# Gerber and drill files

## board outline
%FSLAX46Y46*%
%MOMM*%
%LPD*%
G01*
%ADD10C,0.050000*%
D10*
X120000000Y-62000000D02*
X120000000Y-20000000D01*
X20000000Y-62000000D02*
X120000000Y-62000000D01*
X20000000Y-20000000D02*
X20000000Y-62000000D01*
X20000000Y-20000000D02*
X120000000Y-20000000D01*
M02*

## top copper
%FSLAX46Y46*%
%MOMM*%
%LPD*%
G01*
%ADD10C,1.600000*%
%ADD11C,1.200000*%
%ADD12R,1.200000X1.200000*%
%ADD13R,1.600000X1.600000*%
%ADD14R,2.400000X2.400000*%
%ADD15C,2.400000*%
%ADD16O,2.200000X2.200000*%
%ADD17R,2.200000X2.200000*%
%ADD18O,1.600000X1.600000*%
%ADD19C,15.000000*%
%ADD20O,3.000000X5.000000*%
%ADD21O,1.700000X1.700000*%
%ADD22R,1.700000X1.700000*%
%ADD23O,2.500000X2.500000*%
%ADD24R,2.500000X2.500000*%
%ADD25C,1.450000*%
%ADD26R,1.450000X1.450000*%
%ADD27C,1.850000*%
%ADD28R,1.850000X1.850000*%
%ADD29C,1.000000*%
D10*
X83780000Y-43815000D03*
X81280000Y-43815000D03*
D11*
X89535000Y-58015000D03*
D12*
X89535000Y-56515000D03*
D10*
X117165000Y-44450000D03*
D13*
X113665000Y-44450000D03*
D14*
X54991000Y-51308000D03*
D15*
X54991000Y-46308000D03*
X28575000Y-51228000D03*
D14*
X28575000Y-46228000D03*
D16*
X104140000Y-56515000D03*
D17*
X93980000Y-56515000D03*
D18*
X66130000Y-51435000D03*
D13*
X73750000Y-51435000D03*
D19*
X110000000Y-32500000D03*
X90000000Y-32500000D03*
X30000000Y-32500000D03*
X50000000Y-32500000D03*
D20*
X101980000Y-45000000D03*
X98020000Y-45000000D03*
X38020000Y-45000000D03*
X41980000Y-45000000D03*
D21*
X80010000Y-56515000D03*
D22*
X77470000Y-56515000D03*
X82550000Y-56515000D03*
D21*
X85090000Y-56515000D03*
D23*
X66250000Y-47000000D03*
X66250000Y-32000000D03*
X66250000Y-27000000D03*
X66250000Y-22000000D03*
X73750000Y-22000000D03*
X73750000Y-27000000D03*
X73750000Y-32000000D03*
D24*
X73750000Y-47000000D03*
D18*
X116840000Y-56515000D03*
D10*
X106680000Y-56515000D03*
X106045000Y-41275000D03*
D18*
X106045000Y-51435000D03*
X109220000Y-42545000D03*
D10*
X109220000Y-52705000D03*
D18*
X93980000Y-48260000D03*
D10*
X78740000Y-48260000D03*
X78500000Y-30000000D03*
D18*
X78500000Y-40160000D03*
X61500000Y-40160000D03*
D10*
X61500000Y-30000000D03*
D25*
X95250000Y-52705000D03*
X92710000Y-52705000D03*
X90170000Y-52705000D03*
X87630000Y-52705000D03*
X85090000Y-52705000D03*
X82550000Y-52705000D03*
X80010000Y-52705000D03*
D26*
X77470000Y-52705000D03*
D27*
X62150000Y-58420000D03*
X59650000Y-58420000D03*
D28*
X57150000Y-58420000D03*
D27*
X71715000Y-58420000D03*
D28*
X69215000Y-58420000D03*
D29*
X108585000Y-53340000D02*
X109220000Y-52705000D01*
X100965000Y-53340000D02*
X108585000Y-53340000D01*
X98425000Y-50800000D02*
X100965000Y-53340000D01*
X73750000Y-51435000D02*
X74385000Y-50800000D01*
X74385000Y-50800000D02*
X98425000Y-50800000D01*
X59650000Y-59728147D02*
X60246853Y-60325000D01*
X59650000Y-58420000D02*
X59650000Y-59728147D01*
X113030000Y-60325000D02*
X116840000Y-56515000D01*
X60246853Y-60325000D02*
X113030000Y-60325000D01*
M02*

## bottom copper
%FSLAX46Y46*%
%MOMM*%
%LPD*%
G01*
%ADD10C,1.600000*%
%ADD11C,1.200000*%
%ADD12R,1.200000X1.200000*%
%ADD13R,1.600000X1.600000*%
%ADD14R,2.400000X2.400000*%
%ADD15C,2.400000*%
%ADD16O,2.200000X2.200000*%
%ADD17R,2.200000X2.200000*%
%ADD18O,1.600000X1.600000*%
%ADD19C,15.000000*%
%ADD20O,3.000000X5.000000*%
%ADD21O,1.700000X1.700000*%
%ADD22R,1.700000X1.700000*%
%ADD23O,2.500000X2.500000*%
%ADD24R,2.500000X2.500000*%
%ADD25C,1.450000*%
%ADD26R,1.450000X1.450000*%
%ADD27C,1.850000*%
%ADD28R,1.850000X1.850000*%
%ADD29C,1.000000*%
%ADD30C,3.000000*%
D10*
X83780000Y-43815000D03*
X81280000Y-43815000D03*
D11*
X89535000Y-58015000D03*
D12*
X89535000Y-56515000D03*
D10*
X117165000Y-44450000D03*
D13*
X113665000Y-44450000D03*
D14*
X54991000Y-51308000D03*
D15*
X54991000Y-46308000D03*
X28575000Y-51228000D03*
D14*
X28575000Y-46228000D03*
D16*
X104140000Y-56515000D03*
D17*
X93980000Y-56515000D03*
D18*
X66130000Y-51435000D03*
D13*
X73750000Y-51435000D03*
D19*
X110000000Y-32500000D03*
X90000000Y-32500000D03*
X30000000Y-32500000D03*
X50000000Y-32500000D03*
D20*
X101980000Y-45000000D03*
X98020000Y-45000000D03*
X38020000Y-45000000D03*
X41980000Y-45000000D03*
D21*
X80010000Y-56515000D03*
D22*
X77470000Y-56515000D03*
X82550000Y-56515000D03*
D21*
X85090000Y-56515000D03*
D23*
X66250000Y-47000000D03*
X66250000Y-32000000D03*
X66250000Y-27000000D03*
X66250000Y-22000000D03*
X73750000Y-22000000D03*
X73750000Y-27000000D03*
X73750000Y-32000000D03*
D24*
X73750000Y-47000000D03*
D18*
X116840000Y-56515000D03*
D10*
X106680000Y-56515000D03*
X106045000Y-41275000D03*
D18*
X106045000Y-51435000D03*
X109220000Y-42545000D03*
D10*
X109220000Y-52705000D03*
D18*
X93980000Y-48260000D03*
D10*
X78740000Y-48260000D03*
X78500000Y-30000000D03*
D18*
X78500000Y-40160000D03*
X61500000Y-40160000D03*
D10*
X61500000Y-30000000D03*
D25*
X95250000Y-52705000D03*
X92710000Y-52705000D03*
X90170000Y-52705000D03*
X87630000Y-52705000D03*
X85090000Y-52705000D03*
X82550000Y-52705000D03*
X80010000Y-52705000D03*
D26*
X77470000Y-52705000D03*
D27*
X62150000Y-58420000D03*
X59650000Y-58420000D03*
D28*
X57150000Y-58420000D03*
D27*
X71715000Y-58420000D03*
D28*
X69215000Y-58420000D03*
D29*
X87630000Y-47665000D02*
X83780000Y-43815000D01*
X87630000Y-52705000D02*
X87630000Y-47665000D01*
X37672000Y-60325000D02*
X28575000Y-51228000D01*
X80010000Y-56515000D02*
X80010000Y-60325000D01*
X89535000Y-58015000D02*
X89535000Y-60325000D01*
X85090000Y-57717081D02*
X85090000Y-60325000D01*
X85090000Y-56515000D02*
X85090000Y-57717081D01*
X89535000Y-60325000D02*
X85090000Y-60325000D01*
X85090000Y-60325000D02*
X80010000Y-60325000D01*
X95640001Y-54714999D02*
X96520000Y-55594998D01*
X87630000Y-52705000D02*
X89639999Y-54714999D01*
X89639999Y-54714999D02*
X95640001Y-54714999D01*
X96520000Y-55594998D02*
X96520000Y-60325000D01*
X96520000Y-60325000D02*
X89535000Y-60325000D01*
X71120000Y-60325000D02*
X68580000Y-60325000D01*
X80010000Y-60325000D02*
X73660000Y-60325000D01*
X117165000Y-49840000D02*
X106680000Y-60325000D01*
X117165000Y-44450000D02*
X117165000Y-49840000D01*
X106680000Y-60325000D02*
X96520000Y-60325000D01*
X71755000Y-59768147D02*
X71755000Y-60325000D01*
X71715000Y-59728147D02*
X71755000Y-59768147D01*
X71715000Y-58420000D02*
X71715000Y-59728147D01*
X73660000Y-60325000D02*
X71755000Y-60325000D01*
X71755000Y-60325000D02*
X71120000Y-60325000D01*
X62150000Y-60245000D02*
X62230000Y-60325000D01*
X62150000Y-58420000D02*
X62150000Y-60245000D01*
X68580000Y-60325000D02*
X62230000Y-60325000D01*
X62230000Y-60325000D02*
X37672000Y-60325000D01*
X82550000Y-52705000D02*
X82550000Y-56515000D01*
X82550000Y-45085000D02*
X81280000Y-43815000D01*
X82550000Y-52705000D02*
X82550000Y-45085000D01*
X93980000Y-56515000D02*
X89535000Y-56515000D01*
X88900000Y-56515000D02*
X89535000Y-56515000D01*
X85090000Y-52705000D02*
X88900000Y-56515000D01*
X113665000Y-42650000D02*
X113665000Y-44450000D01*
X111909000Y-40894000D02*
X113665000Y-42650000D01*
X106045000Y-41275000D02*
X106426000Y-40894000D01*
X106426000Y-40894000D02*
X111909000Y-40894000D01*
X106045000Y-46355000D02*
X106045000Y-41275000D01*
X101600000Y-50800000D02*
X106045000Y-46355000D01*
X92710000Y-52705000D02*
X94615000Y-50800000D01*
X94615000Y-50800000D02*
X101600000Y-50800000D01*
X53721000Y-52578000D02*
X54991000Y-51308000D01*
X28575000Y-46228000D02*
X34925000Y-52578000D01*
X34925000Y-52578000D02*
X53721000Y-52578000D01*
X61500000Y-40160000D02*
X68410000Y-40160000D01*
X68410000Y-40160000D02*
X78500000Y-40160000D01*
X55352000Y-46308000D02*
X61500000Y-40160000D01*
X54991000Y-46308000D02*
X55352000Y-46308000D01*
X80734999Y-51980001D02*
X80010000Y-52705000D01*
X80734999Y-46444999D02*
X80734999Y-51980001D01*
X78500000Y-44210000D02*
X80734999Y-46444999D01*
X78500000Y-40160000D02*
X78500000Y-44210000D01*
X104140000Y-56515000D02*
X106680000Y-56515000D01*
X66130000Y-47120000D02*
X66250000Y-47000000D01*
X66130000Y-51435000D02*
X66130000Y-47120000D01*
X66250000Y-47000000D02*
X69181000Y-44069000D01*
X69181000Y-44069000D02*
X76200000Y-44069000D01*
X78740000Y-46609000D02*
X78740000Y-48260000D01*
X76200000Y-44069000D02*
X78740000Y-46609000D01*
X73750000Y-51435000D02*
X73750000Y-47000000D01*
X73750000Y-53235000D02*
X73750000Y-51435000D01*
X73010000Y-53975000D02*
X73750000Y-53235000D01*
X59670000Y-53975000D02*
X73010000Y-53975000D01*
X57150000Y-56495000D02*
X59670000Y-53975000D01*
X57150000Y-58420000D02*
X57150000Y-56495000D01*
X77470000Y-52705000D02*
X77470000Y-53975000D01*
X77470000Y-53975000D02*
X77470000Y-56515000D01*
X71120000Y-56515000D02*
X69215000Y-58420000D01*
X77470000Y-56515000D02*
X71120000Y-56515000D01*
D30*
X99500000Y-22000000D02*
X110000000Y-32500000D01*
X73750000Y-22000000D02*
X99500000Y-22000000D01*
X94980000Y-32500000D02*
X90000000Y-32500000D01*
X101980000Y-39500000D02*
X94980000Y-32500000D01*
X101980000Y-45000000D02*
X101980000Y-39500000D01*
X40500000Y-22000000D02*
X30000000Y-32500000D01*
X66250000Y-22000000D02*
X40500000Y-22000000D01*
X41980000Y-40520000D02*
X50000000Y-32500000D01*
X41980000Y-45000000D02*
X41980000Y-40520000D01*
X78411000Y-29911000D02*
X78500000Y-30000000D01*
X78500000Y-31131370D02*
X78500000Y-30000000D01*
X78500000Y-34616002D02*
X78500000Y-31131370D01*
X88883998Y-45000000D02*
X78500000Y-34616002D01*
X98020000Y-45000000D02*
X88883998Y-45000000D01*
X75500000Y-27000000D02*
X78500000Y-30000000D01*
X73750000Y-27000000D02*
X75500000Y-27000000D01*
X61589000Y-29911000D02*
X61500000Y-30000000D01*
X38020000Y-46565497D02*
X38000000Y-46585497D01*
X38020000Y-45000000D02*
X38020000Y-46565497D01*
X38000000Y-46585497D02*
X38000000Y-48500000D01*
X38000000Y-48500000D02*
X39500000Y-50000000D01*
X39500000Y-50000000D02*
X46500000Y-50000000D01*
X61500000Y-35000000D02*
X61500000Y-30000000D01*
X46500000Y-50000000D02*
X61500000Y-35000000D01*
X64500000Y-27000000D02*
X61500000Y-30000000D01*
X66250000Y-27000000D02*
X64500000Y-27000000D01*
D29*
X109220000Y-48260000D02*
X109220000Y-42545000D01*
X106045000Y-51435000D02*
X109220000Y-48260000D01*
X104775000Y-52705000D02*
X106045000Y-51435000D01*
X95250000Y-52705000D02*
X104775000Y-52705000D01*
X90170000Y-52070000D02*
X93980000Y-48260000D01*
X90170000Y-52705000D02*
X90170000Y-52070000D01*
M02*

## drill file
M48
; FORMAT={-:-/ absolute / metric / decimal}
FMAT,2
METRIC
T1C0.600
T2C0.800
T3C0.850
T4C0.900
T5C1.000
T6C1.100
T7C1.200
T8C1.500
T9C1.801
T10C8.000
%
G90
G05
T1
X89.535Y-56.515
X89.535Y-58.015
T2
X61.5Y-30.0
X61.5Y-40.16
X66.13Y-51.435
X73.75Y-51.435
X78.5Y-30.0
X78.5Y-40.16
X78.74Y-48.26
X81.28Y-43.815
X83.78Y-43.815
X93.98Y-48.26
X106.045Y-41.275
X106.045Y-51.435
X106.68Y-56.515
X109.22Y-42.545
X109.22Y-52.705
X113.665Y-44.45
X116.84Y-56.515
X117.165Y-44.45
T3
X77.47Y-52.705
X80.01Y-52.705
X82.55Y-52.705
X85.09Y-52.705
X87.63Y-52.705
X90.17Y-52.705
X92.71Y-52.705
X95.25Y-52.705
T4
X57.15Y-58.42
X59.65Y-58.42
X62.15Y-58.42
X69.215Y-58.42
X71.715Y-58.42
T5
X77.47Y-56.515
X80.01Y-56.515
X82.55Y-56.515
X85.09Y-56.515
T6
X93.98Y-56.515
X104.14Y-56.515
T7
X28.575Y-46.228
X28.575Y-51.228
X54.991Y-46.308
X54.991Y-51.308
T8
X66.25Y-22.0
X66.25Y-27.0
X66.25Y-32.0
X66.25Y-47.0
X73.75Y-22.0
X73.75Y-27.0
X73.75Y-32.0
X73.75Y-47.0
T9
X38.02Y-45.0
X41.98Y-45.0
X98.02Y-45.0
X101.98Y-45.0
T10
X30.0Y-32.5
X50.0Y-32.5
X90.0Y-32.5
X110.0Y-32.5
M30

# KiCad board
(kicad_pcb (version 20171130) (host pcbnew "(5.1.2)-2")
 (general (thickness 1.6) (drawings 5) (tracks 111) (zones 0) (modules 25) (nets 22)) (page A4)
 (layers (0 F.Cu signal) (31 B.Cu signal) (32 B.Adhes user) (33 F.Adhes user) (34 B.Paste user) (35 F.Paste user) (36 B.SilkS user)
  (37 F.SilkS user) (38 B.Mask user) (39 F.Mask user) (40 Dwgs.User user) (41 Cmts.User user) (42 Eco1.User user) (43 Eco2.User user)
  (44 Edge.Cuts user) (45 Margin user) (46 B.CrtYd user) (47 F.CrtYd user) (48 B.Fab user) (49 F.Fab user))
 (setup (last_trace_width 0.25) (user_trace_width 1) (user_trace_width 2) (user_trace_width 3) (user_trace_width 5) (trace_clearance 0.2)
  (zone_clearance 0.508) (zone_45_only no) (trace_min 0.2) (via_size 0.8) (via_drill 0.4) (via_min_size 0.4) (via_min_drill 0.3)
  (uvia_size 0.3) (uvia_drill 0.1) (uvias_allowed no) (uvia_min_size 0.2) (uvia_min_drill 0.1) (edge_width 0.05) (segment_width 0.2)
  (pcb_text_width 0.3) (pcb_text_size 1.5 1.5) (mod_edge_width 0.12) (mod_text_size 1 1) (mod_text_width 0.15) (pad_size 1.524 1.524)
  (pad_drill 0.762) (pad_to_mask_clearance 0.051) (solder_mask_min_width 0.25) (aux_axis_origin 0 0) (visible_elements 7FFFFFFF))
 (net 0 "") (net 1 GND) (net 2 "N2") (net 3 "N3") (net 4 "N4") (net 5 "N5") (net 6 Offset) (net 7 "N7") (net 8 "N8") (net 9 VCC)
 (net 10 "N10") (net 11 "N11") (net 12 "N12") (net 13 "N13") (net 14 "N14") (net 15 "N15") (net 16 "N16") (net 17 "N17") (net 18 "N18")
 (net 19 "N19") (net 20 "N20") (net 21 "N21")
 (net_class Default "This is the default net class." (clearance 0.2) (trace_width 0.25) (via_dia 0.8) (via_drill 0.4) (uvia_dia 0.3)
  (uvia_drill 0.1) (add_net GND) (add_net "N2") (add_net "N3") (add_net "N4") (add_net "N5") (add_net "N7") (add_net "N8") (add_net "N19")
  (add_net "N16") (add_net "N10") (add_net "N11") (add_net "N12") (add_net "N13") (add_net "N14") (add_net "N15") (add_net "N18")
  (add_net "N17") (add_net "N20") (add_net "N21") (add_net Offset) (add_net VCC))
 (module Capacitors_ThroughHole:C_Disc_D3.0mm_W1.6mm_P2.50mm (layer F.Cu) (at 81.28 43.815)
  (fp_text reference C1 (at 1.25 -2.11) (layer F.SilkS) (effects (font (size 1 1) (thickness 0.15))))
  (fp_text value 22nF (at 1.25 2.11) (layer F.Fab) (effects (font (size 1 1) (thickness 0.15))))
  (pad 2 thru_hole circle (at 2.5 0) (size 1.6 1.6) (drill 0.8) (layers *.Cu *.Mask) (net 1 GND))
  (pad 1 thru_hole circle (at 0 0) (size 1.6 1.6) (drill 0.8) (layers *.Cu *.Mask) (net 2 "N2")))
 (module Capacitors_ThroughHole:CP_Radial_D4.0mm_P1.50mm (layer F.Cu) (at 89.535 56.515 270)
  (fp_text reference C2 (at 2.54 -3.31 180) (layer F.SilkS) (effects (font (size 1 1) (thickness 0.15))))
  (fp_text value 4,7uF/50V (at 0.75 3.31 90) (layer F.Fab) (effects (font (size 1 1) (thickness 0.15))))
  (pad 2 thru_hole circle (at 1.5 0 270) (size 1.2 1.2) (drill 0.6) (layers *.Cu *.Mask) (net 1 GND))
  (pad 1 thru_hole rect (at 0 0 270) (size 1.2 1.2) (drill 0.6) (layers *.Cu *.Mask) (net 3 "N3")))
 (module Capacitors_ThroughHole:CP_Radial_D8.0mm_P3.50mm (layer F.Cu) (at 113.665 44.45)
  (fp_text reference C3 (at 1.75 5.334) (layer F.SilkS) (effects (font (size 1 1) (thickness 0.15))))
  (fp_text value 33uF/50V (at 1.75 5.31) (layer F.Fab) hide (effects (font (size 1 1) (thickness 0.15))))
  (pad 2 thru_hole circle (at 3.5 0) (size 1.6 1.6) (drill 0.8) (layers *.Cu *.Mask) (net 1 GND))
  (pad 1 thru_hole rect (at 0 0) (size 1.6 1.6) (drill 0.8) (layers *.Cu *.Mask) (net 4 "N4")))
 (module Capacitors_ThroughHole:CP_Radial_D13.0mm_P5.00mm (layer F.Cu) (at 54.991 51.308 90)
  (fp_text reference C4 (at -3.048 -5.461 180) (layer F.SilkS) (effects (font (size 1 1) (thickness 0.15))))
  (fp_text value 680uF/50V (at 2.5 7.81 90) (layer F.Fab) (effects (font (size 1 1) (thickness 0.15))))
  (pad 1 thru_hole rect (at 0 0 90) (size 2.4 2.4) (drill 1.2) (layers *.Cu *.Mask) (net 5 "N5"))
  (pad 2 thru_hole circle (at 5 0 90) (size 2.4 2.4) (drill 1.2) (layers *.Cu *.Mask) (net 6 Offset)))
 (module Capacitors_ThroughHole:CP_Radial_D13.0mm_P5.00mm (layer F.Cu) (at 28.575 46.228 270)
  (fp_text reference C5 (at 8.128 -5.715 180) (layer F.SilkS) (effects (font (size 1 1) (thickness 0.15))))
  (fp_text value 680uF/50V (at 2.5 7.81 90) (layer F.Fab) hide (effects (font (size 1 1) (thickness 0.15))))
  (pad 2 thru_hole circle (at 5 0 270) (size 2.4 2.4) (drill 1.2) (layers *.Cu *.Mask) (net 1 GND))
  (pad 1 thru_hole rect (at 0 0 270) (size 2.4 2.4) (drill 1.2) (layers *.Cu *.Mask) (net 5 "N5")))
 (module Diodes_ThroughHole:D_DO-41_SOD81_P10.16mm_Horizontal (layer F.Cu) (at 93.98 56.515)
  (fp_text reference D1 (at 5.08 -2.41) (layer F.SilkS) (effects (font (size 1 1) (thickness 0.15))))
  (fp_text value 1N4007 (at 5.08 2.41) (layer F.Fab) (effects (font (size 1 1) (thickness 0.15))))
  (pad 2 thru_hole oval (at 10.16 0) (size 2.2 2.2) (drill 1.1) (layers *.Cu *.Mask) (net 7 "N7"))
  (pad 1 thru_hole rect (at 0 0) (size 2.2 2.2) (drill 1.1) (layers *.Cu *.Mask) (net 3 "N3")))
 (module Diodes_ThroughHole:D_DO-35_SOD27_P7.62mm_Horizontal (layer F.Cu) (at 73.75 51.435 180)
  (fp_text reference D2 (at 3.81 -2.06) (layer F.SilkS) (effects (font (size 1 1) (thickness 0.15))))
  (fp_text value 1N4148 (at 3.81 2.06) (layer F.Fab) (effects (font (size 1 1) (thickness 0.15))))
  (pad 2 thru_hole oval (at 7.62 0 180) (size 1.6 1.6) (drill 0.8) (layers *.Cu *.Mask) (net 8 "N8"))
  (pad 1 thru_hole rect (at 0 0 180) (size 1.6 1.6) (drill 0.8) (layers *.Cu *.Mask) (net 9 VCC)))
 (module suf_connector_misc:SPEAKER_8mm (layer F.Cu) (at 110 32.5)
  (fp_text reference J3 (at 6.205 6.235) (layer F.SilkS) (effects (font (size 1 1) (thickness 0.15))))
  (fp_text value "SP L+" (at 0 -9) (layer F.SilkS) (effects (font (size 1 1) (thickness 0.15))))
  (pad 1 thru_hole circle (at 0 0) (size 15 15) (drill 8) (layers *.Cu *.Mask) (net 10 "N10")))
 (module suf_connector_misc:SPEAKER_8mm (layer F.Cu) (at 90 32.5)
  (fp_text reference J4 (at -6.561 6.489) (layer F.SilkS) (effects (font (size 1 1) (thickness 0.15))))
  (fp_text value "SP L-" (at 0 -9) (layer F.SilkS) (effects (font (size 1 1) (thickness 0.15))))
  (pad 1 thru_hole circle (at 0 0) (size 15 15) (drill 8) (layers *.Cu *.Mask) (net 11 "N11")))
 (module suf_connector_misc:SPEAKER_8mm (layer F.Cu) (at 30 32.5)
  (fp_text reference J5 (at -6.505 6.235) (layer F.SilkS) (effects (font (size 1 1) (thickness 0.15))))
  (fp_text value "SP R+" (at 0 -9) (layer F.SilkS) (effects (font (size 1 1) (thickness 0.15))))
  (pad 1 thru_hole circle (at 0 0) (size 15 15) (drill 8) (layers *.Cu *.Mask) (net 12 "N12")))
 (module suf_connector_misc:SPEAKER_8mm (layer F.Cu) (at 50 32.5)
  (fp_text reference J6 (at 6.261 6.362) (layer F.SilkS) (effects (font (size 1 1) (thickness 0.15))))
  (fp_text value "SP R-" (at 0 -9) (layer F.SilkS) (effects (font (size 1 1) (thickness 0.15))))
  (pad 1 thru_hole circle (at 0 0) (size 15 15) (drill 8) (layers *.Cu *.Mask) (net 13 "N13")))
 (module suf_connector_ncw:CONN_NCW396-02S (layer F.Cu) (at 100 45)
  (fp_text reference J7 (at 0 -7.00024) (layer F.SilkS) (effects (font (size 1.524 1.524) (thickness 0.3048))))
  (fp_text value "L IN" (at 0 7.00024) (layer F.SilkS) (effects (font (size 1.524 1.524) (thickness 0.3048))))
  (pad 2 thru_hole oval (at 1.98 0) (size 3 5) (drill 1.80086) (layers *.Cu *.Mask F.SilkS) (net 11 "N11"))
  (pad 1 thru_hole oval (at -1.98 0) (size 3 5) (drill 1.80086) (layers *.Cu *.Mask F.SilkS) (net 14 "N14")))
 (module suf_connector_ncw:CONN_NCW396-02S (layer F.Cu) (at 40 45)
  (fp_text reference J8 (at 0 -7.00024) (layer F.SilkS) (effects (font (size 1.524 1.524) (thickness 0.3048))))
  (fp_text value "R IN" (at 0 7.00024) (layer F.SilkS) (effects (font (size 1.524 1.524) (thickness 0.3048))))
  (pad 1 thru_hole oval (at -1.98 0) (size 3 5) (drill 1.80086) (layers *.Cu *.Mask F.SilkS) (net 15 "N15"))
  (pad 2 thru_hole oval (at 1.98 0) (size 3 5) (drill 1.80086) (layers *.Cu *.Mask F.SilkS) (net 13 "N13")))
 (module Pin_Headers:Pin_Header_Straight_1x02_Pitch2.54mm (layer F.Cu) (at 77.47 56.515 90)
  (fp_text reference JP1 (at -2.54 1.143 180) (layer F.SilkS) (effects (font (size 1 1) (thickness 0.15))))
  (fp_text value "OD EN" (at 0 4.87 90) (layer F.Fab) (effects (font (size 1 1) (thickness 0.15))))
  (pad 2 thru_hole oval (at 0 2.54 90) (size 1.7 1.7) (drill 1) (layers *.Cu *.Mask) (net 1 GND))
  (pad 1 thru_hole rect (at 0 0 90) (size 1.7 1.7) (drill 1) (layers *.Cu *.Mask) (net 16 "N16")))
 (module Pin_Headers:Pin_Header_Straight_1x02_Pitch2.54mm (layer F.Cu) (at 82.55 56.515 90)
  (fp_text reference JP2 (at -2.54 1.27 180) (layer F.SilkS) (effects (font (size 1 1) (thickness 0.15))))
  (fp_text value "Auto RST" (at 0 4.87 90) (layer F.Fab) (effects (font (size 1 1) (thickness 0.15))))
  (pad 1 thru_hole rect (at 0 0 90) (size 1.7 1.7) (drill 1) (layers *.Cu *.Mask) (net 2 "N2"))
  (pad 2 thru_hole oval (at 0 2.54 90) (size 1.7 1.7) (drill 1) (layers *.Cu *.Mask) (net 1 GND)))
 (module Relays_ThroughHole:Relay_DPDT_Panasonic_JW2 (layer F.Cu) (at 73.75 47 180)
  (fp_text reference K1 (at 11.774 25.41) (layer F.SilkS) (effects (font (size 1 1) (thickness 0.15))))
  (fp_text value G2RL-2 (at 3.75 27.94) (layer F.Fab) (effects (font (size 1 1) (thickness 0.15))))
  (pad 8 thru_hole oval (at 7.5 0 180) (size 2.5 2.5) (drill 1.5) (layers *.Cu *.Mask) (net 8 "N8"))
  (pad 7 thru_hole oval (at 7.5 15 180) (size 2.5 2.5) (drill 1.5) (layers *.Cu *.Mask) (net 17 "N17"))
  (pad 6 thru_hole oval (at 7.5 20 180) (size 2.5 2.5) (drill 1.5) (layers *.Cu *.Mask) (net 15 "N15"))
  (pad 5 thru_hole oval (at 7.5 25 180) (size 2.5 2.5) (drill 1.5) (layers *.Cu *.Mask) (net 12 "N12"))
  (pad 4 thru_hole oval (at 0 25 180) (size 2.5 2.5) (drill 1.5) (layers *.Cu *.Mask) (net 10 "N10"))
  (pad 3 thru_hole oval (at 0 20 180) (size 2.5 2.5) (drill 1.5) (layers *.Cu *.Mask) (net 14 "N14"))
  (pad 2 thru_hole oval (at 0 15 180) (size 2.5 2.5) (drill 1.5) (layers *.Cu *.Mask) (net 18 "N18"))
  (pad 1 thru_hole rect (at 0 0 180) (size 2.5 2.5) (drill 1.5) (layers *.Cu *.Mask) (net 9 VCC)))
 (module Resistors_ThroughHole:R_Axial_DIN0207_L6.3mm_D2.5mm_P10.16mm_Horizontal (layer F.Cu) (at 106.68 56.515)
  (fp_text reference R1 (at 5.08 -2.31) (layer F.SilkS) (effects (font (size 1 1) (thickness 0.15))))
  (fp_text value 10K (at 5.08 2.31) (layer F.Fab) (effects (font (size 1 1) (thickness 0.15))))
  (pad 2 thru_hole oval (at 10.16 0) (size 1.6 1.6) (drill 0.8) (layers *.Cu *.Mask) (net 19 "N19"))
  (pad 1 thru_hole circle (at 0 0) (size 1.6 1.6) (drill 0.8) (layers *.Cu *.Mask) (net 7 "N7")))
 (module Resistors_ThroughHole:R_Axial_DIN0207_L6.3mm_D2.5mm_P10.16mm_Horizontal (layer F.Cu) (at 106.045 41.275 270)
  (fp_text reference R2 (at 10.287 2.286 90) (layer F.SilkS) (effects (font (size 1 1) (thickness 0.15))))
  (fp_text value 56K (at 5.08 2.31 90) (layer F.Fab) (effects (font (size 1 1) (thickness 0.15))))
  (pad 1 thru_hole circle (at 0 0 270) (size 1.6 1.6) (drill 0.8) (layers *.Cu *.Mask) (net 4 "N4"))
  (pad 2 thru_hole oval (at 10.16 0 270) (size 1.6 1.6) (drill 0.8) (layers *.Cu *.Mask) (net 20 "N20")))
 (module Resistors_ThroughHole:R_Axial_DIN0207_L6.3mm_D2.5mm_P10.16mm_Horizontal (layer F.Cu) (at 109.22 52.705 90)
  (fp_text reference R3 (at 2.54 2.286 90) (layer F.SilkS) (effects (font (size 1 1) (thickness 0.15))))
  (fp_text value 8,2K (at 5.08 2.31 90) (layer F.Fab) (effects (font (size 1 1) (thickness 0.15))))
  (pad 2 thru_hole oval (at 10.16 0 90) (size 1.6 1.6) (drill 0.8) (layers *.Cu *.Mask) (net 20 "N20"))
  (pad 1 thru_hole circle (at 0 0 90) (size 1.6 1.6) (drill 0.8) (layers *.Cu *.Mask) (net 9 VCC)))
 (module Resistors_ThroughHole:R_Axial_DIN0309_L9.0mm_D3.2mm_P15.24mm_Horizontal (layer F.Cu) (at 78.74 48.26)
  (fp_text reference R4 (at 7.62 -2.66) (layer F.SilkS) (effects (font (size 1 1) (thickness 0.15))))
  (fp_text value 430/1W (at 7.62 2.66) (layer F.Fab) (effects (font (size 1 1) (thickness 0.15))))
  (pad 2 thru_hole oval (at 15.24 0) (size 1.6 1.6) (drill 0.8) (layers *.Cu *.Mask) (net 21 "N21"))
  (pad 1 thru_hole circle (at 0 0) (size 1.6 1.6) (drill 0.8) (layers *.Cu *.Mask) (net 8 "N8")))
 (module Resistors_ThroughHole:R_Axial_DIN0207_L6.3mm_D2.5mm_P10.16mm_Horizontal (layer F.Cu) (at 78.5 30 270)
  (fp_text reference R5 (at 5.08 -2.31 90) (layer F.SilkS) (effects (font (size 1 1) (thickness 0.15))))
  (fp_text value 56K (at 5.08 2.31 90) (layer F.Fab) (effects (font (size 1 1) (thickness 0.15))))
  (pad 1 thru_hole circle (at 0 0 270) (size 1.6 1.6) (drill 0.8) (layers *.Cu *.Mask) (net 14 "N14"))
  (pad 2 thru_hole oval (at 10.16 0 270) (size 1.6 1.6) (drill 0.8) (layers *.Cu *.Mask) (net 6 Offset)))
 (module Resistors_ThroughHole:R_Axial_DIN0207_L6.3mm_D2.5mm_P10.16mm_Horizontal (layer F.Cu) (at 61.5 30 270)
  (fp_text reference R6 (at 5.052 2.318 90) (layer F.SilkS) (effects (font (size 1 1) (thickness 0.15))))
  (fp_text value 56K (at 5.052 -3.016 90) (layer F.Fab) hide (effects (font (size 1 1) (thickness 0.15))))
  (pad 2 thru_hole oval (at 10.16 0 270) (size 1.6 1.6) (drill 0.8) (layers *.Cu *.Mask) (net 6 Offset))
  (pad 1 thru_hole circle (at 0 0 270) (size 1.6 1.6) (drill 0.8) (layers *.Cu *.Mask) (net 15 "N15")))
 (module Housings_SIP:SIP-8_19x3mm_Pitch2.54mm (layer F.Cu) (at 77.47 52.705)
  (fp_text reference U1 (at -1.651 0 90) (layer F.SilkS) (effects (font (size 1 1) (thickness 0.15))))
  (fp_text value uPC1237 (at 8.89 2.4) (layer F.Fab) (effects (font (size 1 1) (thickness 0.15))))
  (pad 8 thru_hole circle (at 17.78 0 90) (size 1.45 1.45) (drill 0.85) (layers *.Cu *.Mask) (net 20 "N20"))
  (pad 7 thru_hole circle (at 15.24 0 90) (size 1.45 1.45) (drill 0.85) (layers *.Cu *.Mask) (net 4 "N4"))
  (pad 6 thru_hole circle (at 12.7 0 90) (size 1.45 1.45) (drill 0.85) (layers *.Cu *.Mask) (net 21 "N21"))
  (pad 5 thru_hole circle (at 10.16 0 90) (size 1.45 1.45) (drill 0.85) (layers *.Cu *.Mask) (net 1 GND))
  (pad 4 thru_hole circle (at 7.62 0 90) (size 1.45 1.45) (drill 0.85) (layers *.Cu *.Mask) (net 3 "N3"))
  (pad 3 thru_hole circle (at 5.08 0 90) (size 1.45 1.45) (drill 0.85) (layers *.Cu *.Mask) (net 2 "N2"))
  (pad 2 thru_hole circle (at 2.54 0 90) (size 1.45 1.45) (drill 0.85) (layers *.Cu *.Mask) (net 6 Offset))
  (pad 1 thru_hole rect (at 0 0 90) (size 1.45 1.45) (drill 0.85) (layers *.Cu *.Mask) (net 16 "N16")))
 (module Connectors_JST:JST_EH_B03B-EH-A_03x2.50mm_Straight (layer F.Cu) (at 57.15 58.42)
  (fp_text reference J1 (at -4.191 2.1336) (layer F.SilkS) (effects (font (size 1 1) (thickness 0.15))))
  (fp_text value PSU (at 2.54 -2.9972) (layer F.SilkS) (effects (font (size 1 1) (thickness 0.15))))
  (pad 3 thru_hole circle (at 5 0) (size 1.85 1.85) (drill 0.9) (layers *.Cu *.Mask) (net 1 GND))
  (pad 2 thru_hole circle (at 2.5 0) (size 1.85 1.85) (drill 0.9) (layers *.Cu *.Mask) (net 19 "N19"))
  (pad 1 thru_hole rect (at 0 0) (size 1.85 1.85) (drill 0.9) (layers *.Cu *.Mask) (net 9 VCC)))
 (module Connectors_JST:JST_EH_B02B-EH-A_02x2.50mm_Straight (layer F.Cu) (at 69.215 58.42)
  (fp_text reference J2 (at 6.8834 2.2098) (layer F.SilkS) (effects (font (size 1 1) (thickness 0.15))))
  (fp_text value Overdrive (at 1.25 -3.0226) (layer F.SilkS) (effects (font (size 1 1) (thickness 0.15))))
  (pad 2 thru_hole circle (at 2.5 0) (size 1.85 1.85) (drill 0.9) (layers *.Cu *.Mask) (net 1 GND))
  (pad 1 thru_hole rect (at 0 0) (size 1.85 1.85) (drill 0.9) (layers *.Cu *.Mask) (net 16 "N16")))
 (gr_line (start 120 62) (end 120 20) (layer Edge.Cuts) (width 0.05))
 (gr_line (start 20 62) (end 120 62) (layer Edge.Cuts) (width 0.05))
 (gr_line (start 20 20) (end 20 62) (layer Edge.Cuts) (width 0.05))
 (gr_line (start 20 20) (end 120 20) (layer Edge.Cuts) (width 0.05))
 (segment (start 87.63 47.665) (end 83.78 43.815) (width 1) (layer B.Cu) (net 1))
 (segment (start 87.63 52.705) (end 87.63 47.665) (width 1) (layer B.Cu) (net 1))
 (segment (start 37.672 60.325) (end 28.575 51.228) (width 1) (layer B.Cu) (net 1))
 (segment (start 80.01 56.515) (end 80.01 60.325) (width 1) (layer B.Cu) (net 1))
 (segment (start 89.535 58.015) (end 89.535 60.325) (width 1) (layer B.Cu) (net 1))
 (segment (start 85.09 57.717081) (end 85.09 60.325) (width 1) (layer B.Cu) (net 1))
 (segment (start 85.09 56.515) (end 85.09 57.717081) (width 1) (layer B.Cu) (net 1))
 (segment (start 89.535 60.325) (end 85.09 60.325) (width 1) (layer B.Cu) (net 1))
 (segment (start 85.09 60.325) (end 80.01 60.325) (width 1) (layer B.Cu) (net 1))
 (segment (start 95.640001 54.714999) (end 96.52 55.594998) (width 1) (layer B.Cu) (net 1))
 (segment (start 87.63 52.705) (end 89.639999 54.714999) (width 1) (layer B.Cu) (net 1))
 (segment (start 89.639999 54.714999) (end 95.640001 54.714999) (width 1) (layer B.Cu) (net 1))
 (segment (start 96.52 55.594998) (end 96.52 60.325) (width 1) (layer B.Cu) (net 1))
 (segment (start 96.52 60.325) (end 89.535 60.325) (width 1) (layer B.Cu) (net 1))
 (segment (start 71.12 60.325) (end 68.58 60.325) (width 1) (layer B.Cu) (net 1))
 (segment (start 80.01 60.325) (end 73.66 60.325) (width 1) (layer B.Cu) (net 1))
 (segment (start 117.165 49.84) (end 106.68 60.325) (width 1) (layer B.Cu) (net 1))
 (segment (start 117.165 44.45) (end 117.165 49.84) (width 1) (layer B.Cu) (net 1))
 (segment (start 106.68 60.325) (end 96.52 60.325) (width 1) (layer B.Cu) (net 1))
 (segment (start 71.755 59.768147) (end 71.755 60.325) (width 1) (layer B.Cu) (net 1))
 (segment (start 71.715 59.728147) (end 71.755 59.768147) (width 1) (layer B.Cu) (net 1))
 (segment (start 71.715 58.42) (end 71.715 59.728147) (width 1) (layer B.Cu) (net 1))
 (segment (start 73.66 60.325) (end 71.755 60.325) (width 1) (layer B.Cu) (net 1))
 (segment (start 71.755 60.325) (end 71.12 60.325) (width 1) (layer B.Cu) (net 1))
 (segment (start 62.15 60.245) (end 62.23 60.325) (width 1) (layer B.Cu) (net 1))
 (segment (start 62.15 58.42) (end 62.15 60.245) (width 1) (layer B.Cu) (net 1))
 (segment (start 68.58 60.325) (end 62.23 60.325) (width 1) (layer B.Cu) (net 1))
 (segment (start 62.23 60.325) (end 37.672 60.325) (width 1) (layer B.Cu) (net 1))
 (segment (start 82.55 52.705) (end 82.55 56.515) (width 1) (layer B.Cu) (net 2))
 (segment (start 82.55 45.085) (end 81.28 43.815) (width 1) (layer B.Cu) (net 2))
 (segment (start 82.55 52.705) (end 82.55 45.085) (width 1) (layer B.Cu) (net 2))
 (segment (start 93.98 56.515) (end 89.535 56.515) (width 1) (layer B.Cu) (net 3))
 (segment (start 88.9 56.515) (end 89.535 56.515) (width 1) (layer B.Cu) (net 3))
 (segment (start 85.09 52.705) (end 88.9 56.515) (width 1) (layer B.Cu) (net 3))
 (segment (start 113.665 42.65) (end 113.665 44.45) (width 1) (layer B.Cu) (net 4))
 (segment (start 111.909 40.894) (end 113.665 42.65) (width 1) (layer B.Cu) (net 4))
 (segment (start 106.045 41.275) (end 106.426 40.894) (width 1) (layer B.Cu) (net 4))
 (segment (start 106.426 40.894) (end 111.909 40.894) (width 1) (layer B.Cu) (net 4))
 (segment (start 106.045 46.355) (end 106.045 41.275) (width 1) (layer B.Cu) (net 4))
 (segment (start 101.6 50.8) (end 106.045 46.355) (width 1) (layer B.Cu) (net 4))
 (segment (start 92.71 52.705) (end 94.615 50.8) (width 1) (layer B.Cu) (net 4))
 (segment (start 94.615 50.8) (end 101.6 50.8) (width 1) (layer B.Cu) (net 4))
 (segment (start 53.721 52.578) (end 54.991 51.308) (width 1) (layer B.Cu) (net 5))
 (segment (start 28.575 46.228) (end 34.925 52.578) (width 1) (layer B.Cu) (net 5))
 (segment (start 34.925 52.578) (end 53.721 52.578) (width 1) (layer B.Cu) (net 5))
 (segment (start 61.5 40.16) (end 68.41 40.16) (width 1) (layer B.Cu) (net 6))
 (segment (start 68.41 40.16) (end 78.5 40.16) (width 1) (layer B.Cu) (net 6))
 (segment (start 55.352 46.308) (end 61.5 40.16) (width 1) (layer B.Cu) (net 6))
 (segment (start 54.991 46.308) (end 55.352 46.308) (width 1) (layer B.Cu) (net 6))
 (segment (start 80.734999 51.980001) (end 80.01 52.705) (width 1) (layer B.Cu) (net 6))
 (segment (start 80.734999 46.444999) (end 80.734999 51.980001) (width 1) (layer B.Cu) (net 6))
 (segment (start 78.5 44.21) (end 80.734999 46.444999) (width 1) (layer B.Cu) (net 6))
 (segment (start 78.5 40.16) (end 78.5 44.21) (width 1) (layer B.Cu) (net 6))
 (segment (start 104.14 56.515) (end 106.68 56.515) (width 1) (layer B.Cu) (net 7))
 (segment (start 66.13 47.12) (end 66.25 47) (width 1) (layer B.Cu) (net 8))
 (segment (start 66.13 51.435) (end 66.13 47.12) (width 1) (layer B.Cu) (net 8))
 (segment (start 66.25 47) (end 69.181 44.069) (width 1) (layer B.Cu) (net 8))
 (segment (start 69.181 44.069) (end 76.2 44.069) (width 1) (layer B.Cu) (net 8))
 (segment (start 78.74 46.609) (end 78.74 48.26) (width 1) (layer B.Cu) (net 8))
 (segment (start 76.2 44.069) (end 78.74 46.609) (width 1) (layer B.Cu) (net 8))
 (segment (start 73.75 51.435) (end 73.75 47) (width 1) (layer B.Cu) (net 9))
 (segment (start 108.585 53.34) (end 109.22 52.705) (width 1) (layer F.Cu) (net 9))
 (segment (start 100.965 53.34) (end 108.585 53.34) (width 1) (layer F.Cu) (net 9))
 (segment (start 98.425 50.8) (end 100.965 53.34) (width 1) (layer F.Cu) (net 9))
 (segment (start 73.75 51.435) (end 74.385 50.8) (width 1) (layer F.Cu) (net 9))
 (segment (start 74.385 50.8) (end 98.425 50.8) (width 1) (layer F.Cu) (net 9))
 (segment (start 73.75 53.235) (end 73.75 51.435) (width 1) (layer B.Cu) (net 9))
 (segment (start 73.01 53.975) (end 73.75 53.235) (width 1) (layer B.Cu) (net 9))
 (segment (start 59.67 53.975) (end 73.01 53.975) (width 1) (layer B.Cu) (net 9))
 (segment (start 57.15 56.495) (end 59.67 53.975) (width 1) (layer B.Cu) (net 9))
 (segment (start 57.15 58.42) (end 57.15 56.495) (width 1) (layer B.Cu) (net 9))
 (segment (start 59.65 59.728147) (end 60.246853 60.325) (width 1) (layer F.Cu) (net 19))
 (segment (start 59.65 58.42) (end 59.65 59.728147) (width 1) (layer F.Cu) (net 19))
 (segment (start 113.03 60.325) (end 116.84 56.515) (width 1) (layer F.Cu) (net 19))
 (segment (start 60.246853 60.325) (end 113.03 60.325) (width 1) (layer F.Cu) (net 19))
 (segment (start 77.47 52.705) (end 77.47 53.975) (width 1) (layer B.Cu) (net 16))
 (segment (start 77.47 53.975) (end 77.47 56.515) (width 1) (layer B.Cu) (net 16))
 (segment (start 71.12 56.515) (end 69.215 58.42) (width 1) (layer B.Cu) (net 16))
 (segment (start 77.47 56.515) (end 71.12 56.515) (width 1) (layer B.Cu) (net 16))
 (segment (start 99.5 22) (end 110 32.5) (width 3) (layer B.Cu) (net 10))
 (segment (start 73.75 22) (end 99.5 22) (width 3) (layer B.Cu) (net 10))
 (segment (start 94.98 32.5) (end 90 32.5) (width 3) (layer B.Cu) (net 11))
 (segment (start 101.98 39.5) (end 94.98 32.5) (width 3) (layer B.Cu) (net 11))
 (segment (start 101.98 45) (end 101.98 39.5) (width 3) (layer B.Cu) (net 11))
 (segment (start 40.5 22) (end 30 32.5) (width 3) (layer B.Cu) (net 12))
 (segment (start 66.25 22) (end 40.5 22) (width 3) (layer B.Cu) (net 12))
 (segment (start 41.98 40.52) (end 50 32.5) (width 3) (layer B.Cu) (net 13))
 (segment (start 41.98 45) (end 41.98 40.52) (width 3) (layer B.Cu) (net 13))
 (segment (start 78.411 29.911) (end 78.5 30) (width 3) (layer B.Cu) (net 14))
 (segment (start 78.5 31.13137) (end 78.5 30) (width 3) (layer B.Cu) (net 14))
 (segment (start 78.5 34.616002) (end 78.5 31.13137) (width 3) (layer B.Cu) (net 14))
 (segment (start 88.883998 45) (end 78.5 34.616002) (width 3) (layer B.Cu) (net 14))
 (segment (start 98.02 45) (end 88.883998 45) (width 3) (layer B.Cu) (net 14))
 (segment (start 75.5 27) (end 78.5 30) (width 3) (layer B.Cu) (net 14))
 (segment (start 73.75 27) (end 75.5 27) (width 3) (layer B.Cu) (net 14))
 (segment (start 61.589 29.911) (end 61.5 30) (width 3) (layer B.Cu) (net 15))
 (segment (start 38.02 46.565497) (end 38 46.585497) (width 3) (layer B.Cu) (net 15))
 (segment (start 38.02 45) (end 38.02 46.565497) (width 3) (layer B.Cu) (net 15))
 (segment (start 38 46.585497) (end 38 48.5) (width 3) (layer B.Cu) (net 15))
 (segment (start 38 48.5) (end 39.5 50) (width 3) (layer B.Cu) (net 15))
 (segment (start 39.5 50) (end 46.5 50) (width 3) (layer B.Cu) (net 15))
 (segment (start 61.5 35) (end 61.5 30) (width 3) (layer B.Cu) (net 15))
 (segment (start 46.5 50) (end 61.5 35) (width 3) (layer B.Cu) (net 15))
 (segment (start 64.5 27) (end 61.5 30) (width 3) (layer B.Cu) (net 15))
 (segment (start 66.25 27) (end 64.5 27) (width 3) (layer B.Cu) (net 15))
 (segment (start 109.22 48.26) (end 109.22 42.545) (width 1) (layer B.Cu) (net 20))
 (segment (start 106.045 51.435) (end 109.22 48.26) (width 1) (layer B.Cu) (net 20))
 (segment (start 104.775 52.705) (end 106.045 51.435) (width 1) (layer B.Cu) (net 20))
 (segment (start 95.25 52.705) (end 104.775 52.705) (width 1) (layer B.Cu) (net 20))
 (segment (start 90.17 52.07) (end 93.98 48.26) (width 1) (layer B.Cu) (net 21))
 (segment (start 90.17 52.705) (end 90.17 52.07) (width 1) (layer B.Cu) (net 21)))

